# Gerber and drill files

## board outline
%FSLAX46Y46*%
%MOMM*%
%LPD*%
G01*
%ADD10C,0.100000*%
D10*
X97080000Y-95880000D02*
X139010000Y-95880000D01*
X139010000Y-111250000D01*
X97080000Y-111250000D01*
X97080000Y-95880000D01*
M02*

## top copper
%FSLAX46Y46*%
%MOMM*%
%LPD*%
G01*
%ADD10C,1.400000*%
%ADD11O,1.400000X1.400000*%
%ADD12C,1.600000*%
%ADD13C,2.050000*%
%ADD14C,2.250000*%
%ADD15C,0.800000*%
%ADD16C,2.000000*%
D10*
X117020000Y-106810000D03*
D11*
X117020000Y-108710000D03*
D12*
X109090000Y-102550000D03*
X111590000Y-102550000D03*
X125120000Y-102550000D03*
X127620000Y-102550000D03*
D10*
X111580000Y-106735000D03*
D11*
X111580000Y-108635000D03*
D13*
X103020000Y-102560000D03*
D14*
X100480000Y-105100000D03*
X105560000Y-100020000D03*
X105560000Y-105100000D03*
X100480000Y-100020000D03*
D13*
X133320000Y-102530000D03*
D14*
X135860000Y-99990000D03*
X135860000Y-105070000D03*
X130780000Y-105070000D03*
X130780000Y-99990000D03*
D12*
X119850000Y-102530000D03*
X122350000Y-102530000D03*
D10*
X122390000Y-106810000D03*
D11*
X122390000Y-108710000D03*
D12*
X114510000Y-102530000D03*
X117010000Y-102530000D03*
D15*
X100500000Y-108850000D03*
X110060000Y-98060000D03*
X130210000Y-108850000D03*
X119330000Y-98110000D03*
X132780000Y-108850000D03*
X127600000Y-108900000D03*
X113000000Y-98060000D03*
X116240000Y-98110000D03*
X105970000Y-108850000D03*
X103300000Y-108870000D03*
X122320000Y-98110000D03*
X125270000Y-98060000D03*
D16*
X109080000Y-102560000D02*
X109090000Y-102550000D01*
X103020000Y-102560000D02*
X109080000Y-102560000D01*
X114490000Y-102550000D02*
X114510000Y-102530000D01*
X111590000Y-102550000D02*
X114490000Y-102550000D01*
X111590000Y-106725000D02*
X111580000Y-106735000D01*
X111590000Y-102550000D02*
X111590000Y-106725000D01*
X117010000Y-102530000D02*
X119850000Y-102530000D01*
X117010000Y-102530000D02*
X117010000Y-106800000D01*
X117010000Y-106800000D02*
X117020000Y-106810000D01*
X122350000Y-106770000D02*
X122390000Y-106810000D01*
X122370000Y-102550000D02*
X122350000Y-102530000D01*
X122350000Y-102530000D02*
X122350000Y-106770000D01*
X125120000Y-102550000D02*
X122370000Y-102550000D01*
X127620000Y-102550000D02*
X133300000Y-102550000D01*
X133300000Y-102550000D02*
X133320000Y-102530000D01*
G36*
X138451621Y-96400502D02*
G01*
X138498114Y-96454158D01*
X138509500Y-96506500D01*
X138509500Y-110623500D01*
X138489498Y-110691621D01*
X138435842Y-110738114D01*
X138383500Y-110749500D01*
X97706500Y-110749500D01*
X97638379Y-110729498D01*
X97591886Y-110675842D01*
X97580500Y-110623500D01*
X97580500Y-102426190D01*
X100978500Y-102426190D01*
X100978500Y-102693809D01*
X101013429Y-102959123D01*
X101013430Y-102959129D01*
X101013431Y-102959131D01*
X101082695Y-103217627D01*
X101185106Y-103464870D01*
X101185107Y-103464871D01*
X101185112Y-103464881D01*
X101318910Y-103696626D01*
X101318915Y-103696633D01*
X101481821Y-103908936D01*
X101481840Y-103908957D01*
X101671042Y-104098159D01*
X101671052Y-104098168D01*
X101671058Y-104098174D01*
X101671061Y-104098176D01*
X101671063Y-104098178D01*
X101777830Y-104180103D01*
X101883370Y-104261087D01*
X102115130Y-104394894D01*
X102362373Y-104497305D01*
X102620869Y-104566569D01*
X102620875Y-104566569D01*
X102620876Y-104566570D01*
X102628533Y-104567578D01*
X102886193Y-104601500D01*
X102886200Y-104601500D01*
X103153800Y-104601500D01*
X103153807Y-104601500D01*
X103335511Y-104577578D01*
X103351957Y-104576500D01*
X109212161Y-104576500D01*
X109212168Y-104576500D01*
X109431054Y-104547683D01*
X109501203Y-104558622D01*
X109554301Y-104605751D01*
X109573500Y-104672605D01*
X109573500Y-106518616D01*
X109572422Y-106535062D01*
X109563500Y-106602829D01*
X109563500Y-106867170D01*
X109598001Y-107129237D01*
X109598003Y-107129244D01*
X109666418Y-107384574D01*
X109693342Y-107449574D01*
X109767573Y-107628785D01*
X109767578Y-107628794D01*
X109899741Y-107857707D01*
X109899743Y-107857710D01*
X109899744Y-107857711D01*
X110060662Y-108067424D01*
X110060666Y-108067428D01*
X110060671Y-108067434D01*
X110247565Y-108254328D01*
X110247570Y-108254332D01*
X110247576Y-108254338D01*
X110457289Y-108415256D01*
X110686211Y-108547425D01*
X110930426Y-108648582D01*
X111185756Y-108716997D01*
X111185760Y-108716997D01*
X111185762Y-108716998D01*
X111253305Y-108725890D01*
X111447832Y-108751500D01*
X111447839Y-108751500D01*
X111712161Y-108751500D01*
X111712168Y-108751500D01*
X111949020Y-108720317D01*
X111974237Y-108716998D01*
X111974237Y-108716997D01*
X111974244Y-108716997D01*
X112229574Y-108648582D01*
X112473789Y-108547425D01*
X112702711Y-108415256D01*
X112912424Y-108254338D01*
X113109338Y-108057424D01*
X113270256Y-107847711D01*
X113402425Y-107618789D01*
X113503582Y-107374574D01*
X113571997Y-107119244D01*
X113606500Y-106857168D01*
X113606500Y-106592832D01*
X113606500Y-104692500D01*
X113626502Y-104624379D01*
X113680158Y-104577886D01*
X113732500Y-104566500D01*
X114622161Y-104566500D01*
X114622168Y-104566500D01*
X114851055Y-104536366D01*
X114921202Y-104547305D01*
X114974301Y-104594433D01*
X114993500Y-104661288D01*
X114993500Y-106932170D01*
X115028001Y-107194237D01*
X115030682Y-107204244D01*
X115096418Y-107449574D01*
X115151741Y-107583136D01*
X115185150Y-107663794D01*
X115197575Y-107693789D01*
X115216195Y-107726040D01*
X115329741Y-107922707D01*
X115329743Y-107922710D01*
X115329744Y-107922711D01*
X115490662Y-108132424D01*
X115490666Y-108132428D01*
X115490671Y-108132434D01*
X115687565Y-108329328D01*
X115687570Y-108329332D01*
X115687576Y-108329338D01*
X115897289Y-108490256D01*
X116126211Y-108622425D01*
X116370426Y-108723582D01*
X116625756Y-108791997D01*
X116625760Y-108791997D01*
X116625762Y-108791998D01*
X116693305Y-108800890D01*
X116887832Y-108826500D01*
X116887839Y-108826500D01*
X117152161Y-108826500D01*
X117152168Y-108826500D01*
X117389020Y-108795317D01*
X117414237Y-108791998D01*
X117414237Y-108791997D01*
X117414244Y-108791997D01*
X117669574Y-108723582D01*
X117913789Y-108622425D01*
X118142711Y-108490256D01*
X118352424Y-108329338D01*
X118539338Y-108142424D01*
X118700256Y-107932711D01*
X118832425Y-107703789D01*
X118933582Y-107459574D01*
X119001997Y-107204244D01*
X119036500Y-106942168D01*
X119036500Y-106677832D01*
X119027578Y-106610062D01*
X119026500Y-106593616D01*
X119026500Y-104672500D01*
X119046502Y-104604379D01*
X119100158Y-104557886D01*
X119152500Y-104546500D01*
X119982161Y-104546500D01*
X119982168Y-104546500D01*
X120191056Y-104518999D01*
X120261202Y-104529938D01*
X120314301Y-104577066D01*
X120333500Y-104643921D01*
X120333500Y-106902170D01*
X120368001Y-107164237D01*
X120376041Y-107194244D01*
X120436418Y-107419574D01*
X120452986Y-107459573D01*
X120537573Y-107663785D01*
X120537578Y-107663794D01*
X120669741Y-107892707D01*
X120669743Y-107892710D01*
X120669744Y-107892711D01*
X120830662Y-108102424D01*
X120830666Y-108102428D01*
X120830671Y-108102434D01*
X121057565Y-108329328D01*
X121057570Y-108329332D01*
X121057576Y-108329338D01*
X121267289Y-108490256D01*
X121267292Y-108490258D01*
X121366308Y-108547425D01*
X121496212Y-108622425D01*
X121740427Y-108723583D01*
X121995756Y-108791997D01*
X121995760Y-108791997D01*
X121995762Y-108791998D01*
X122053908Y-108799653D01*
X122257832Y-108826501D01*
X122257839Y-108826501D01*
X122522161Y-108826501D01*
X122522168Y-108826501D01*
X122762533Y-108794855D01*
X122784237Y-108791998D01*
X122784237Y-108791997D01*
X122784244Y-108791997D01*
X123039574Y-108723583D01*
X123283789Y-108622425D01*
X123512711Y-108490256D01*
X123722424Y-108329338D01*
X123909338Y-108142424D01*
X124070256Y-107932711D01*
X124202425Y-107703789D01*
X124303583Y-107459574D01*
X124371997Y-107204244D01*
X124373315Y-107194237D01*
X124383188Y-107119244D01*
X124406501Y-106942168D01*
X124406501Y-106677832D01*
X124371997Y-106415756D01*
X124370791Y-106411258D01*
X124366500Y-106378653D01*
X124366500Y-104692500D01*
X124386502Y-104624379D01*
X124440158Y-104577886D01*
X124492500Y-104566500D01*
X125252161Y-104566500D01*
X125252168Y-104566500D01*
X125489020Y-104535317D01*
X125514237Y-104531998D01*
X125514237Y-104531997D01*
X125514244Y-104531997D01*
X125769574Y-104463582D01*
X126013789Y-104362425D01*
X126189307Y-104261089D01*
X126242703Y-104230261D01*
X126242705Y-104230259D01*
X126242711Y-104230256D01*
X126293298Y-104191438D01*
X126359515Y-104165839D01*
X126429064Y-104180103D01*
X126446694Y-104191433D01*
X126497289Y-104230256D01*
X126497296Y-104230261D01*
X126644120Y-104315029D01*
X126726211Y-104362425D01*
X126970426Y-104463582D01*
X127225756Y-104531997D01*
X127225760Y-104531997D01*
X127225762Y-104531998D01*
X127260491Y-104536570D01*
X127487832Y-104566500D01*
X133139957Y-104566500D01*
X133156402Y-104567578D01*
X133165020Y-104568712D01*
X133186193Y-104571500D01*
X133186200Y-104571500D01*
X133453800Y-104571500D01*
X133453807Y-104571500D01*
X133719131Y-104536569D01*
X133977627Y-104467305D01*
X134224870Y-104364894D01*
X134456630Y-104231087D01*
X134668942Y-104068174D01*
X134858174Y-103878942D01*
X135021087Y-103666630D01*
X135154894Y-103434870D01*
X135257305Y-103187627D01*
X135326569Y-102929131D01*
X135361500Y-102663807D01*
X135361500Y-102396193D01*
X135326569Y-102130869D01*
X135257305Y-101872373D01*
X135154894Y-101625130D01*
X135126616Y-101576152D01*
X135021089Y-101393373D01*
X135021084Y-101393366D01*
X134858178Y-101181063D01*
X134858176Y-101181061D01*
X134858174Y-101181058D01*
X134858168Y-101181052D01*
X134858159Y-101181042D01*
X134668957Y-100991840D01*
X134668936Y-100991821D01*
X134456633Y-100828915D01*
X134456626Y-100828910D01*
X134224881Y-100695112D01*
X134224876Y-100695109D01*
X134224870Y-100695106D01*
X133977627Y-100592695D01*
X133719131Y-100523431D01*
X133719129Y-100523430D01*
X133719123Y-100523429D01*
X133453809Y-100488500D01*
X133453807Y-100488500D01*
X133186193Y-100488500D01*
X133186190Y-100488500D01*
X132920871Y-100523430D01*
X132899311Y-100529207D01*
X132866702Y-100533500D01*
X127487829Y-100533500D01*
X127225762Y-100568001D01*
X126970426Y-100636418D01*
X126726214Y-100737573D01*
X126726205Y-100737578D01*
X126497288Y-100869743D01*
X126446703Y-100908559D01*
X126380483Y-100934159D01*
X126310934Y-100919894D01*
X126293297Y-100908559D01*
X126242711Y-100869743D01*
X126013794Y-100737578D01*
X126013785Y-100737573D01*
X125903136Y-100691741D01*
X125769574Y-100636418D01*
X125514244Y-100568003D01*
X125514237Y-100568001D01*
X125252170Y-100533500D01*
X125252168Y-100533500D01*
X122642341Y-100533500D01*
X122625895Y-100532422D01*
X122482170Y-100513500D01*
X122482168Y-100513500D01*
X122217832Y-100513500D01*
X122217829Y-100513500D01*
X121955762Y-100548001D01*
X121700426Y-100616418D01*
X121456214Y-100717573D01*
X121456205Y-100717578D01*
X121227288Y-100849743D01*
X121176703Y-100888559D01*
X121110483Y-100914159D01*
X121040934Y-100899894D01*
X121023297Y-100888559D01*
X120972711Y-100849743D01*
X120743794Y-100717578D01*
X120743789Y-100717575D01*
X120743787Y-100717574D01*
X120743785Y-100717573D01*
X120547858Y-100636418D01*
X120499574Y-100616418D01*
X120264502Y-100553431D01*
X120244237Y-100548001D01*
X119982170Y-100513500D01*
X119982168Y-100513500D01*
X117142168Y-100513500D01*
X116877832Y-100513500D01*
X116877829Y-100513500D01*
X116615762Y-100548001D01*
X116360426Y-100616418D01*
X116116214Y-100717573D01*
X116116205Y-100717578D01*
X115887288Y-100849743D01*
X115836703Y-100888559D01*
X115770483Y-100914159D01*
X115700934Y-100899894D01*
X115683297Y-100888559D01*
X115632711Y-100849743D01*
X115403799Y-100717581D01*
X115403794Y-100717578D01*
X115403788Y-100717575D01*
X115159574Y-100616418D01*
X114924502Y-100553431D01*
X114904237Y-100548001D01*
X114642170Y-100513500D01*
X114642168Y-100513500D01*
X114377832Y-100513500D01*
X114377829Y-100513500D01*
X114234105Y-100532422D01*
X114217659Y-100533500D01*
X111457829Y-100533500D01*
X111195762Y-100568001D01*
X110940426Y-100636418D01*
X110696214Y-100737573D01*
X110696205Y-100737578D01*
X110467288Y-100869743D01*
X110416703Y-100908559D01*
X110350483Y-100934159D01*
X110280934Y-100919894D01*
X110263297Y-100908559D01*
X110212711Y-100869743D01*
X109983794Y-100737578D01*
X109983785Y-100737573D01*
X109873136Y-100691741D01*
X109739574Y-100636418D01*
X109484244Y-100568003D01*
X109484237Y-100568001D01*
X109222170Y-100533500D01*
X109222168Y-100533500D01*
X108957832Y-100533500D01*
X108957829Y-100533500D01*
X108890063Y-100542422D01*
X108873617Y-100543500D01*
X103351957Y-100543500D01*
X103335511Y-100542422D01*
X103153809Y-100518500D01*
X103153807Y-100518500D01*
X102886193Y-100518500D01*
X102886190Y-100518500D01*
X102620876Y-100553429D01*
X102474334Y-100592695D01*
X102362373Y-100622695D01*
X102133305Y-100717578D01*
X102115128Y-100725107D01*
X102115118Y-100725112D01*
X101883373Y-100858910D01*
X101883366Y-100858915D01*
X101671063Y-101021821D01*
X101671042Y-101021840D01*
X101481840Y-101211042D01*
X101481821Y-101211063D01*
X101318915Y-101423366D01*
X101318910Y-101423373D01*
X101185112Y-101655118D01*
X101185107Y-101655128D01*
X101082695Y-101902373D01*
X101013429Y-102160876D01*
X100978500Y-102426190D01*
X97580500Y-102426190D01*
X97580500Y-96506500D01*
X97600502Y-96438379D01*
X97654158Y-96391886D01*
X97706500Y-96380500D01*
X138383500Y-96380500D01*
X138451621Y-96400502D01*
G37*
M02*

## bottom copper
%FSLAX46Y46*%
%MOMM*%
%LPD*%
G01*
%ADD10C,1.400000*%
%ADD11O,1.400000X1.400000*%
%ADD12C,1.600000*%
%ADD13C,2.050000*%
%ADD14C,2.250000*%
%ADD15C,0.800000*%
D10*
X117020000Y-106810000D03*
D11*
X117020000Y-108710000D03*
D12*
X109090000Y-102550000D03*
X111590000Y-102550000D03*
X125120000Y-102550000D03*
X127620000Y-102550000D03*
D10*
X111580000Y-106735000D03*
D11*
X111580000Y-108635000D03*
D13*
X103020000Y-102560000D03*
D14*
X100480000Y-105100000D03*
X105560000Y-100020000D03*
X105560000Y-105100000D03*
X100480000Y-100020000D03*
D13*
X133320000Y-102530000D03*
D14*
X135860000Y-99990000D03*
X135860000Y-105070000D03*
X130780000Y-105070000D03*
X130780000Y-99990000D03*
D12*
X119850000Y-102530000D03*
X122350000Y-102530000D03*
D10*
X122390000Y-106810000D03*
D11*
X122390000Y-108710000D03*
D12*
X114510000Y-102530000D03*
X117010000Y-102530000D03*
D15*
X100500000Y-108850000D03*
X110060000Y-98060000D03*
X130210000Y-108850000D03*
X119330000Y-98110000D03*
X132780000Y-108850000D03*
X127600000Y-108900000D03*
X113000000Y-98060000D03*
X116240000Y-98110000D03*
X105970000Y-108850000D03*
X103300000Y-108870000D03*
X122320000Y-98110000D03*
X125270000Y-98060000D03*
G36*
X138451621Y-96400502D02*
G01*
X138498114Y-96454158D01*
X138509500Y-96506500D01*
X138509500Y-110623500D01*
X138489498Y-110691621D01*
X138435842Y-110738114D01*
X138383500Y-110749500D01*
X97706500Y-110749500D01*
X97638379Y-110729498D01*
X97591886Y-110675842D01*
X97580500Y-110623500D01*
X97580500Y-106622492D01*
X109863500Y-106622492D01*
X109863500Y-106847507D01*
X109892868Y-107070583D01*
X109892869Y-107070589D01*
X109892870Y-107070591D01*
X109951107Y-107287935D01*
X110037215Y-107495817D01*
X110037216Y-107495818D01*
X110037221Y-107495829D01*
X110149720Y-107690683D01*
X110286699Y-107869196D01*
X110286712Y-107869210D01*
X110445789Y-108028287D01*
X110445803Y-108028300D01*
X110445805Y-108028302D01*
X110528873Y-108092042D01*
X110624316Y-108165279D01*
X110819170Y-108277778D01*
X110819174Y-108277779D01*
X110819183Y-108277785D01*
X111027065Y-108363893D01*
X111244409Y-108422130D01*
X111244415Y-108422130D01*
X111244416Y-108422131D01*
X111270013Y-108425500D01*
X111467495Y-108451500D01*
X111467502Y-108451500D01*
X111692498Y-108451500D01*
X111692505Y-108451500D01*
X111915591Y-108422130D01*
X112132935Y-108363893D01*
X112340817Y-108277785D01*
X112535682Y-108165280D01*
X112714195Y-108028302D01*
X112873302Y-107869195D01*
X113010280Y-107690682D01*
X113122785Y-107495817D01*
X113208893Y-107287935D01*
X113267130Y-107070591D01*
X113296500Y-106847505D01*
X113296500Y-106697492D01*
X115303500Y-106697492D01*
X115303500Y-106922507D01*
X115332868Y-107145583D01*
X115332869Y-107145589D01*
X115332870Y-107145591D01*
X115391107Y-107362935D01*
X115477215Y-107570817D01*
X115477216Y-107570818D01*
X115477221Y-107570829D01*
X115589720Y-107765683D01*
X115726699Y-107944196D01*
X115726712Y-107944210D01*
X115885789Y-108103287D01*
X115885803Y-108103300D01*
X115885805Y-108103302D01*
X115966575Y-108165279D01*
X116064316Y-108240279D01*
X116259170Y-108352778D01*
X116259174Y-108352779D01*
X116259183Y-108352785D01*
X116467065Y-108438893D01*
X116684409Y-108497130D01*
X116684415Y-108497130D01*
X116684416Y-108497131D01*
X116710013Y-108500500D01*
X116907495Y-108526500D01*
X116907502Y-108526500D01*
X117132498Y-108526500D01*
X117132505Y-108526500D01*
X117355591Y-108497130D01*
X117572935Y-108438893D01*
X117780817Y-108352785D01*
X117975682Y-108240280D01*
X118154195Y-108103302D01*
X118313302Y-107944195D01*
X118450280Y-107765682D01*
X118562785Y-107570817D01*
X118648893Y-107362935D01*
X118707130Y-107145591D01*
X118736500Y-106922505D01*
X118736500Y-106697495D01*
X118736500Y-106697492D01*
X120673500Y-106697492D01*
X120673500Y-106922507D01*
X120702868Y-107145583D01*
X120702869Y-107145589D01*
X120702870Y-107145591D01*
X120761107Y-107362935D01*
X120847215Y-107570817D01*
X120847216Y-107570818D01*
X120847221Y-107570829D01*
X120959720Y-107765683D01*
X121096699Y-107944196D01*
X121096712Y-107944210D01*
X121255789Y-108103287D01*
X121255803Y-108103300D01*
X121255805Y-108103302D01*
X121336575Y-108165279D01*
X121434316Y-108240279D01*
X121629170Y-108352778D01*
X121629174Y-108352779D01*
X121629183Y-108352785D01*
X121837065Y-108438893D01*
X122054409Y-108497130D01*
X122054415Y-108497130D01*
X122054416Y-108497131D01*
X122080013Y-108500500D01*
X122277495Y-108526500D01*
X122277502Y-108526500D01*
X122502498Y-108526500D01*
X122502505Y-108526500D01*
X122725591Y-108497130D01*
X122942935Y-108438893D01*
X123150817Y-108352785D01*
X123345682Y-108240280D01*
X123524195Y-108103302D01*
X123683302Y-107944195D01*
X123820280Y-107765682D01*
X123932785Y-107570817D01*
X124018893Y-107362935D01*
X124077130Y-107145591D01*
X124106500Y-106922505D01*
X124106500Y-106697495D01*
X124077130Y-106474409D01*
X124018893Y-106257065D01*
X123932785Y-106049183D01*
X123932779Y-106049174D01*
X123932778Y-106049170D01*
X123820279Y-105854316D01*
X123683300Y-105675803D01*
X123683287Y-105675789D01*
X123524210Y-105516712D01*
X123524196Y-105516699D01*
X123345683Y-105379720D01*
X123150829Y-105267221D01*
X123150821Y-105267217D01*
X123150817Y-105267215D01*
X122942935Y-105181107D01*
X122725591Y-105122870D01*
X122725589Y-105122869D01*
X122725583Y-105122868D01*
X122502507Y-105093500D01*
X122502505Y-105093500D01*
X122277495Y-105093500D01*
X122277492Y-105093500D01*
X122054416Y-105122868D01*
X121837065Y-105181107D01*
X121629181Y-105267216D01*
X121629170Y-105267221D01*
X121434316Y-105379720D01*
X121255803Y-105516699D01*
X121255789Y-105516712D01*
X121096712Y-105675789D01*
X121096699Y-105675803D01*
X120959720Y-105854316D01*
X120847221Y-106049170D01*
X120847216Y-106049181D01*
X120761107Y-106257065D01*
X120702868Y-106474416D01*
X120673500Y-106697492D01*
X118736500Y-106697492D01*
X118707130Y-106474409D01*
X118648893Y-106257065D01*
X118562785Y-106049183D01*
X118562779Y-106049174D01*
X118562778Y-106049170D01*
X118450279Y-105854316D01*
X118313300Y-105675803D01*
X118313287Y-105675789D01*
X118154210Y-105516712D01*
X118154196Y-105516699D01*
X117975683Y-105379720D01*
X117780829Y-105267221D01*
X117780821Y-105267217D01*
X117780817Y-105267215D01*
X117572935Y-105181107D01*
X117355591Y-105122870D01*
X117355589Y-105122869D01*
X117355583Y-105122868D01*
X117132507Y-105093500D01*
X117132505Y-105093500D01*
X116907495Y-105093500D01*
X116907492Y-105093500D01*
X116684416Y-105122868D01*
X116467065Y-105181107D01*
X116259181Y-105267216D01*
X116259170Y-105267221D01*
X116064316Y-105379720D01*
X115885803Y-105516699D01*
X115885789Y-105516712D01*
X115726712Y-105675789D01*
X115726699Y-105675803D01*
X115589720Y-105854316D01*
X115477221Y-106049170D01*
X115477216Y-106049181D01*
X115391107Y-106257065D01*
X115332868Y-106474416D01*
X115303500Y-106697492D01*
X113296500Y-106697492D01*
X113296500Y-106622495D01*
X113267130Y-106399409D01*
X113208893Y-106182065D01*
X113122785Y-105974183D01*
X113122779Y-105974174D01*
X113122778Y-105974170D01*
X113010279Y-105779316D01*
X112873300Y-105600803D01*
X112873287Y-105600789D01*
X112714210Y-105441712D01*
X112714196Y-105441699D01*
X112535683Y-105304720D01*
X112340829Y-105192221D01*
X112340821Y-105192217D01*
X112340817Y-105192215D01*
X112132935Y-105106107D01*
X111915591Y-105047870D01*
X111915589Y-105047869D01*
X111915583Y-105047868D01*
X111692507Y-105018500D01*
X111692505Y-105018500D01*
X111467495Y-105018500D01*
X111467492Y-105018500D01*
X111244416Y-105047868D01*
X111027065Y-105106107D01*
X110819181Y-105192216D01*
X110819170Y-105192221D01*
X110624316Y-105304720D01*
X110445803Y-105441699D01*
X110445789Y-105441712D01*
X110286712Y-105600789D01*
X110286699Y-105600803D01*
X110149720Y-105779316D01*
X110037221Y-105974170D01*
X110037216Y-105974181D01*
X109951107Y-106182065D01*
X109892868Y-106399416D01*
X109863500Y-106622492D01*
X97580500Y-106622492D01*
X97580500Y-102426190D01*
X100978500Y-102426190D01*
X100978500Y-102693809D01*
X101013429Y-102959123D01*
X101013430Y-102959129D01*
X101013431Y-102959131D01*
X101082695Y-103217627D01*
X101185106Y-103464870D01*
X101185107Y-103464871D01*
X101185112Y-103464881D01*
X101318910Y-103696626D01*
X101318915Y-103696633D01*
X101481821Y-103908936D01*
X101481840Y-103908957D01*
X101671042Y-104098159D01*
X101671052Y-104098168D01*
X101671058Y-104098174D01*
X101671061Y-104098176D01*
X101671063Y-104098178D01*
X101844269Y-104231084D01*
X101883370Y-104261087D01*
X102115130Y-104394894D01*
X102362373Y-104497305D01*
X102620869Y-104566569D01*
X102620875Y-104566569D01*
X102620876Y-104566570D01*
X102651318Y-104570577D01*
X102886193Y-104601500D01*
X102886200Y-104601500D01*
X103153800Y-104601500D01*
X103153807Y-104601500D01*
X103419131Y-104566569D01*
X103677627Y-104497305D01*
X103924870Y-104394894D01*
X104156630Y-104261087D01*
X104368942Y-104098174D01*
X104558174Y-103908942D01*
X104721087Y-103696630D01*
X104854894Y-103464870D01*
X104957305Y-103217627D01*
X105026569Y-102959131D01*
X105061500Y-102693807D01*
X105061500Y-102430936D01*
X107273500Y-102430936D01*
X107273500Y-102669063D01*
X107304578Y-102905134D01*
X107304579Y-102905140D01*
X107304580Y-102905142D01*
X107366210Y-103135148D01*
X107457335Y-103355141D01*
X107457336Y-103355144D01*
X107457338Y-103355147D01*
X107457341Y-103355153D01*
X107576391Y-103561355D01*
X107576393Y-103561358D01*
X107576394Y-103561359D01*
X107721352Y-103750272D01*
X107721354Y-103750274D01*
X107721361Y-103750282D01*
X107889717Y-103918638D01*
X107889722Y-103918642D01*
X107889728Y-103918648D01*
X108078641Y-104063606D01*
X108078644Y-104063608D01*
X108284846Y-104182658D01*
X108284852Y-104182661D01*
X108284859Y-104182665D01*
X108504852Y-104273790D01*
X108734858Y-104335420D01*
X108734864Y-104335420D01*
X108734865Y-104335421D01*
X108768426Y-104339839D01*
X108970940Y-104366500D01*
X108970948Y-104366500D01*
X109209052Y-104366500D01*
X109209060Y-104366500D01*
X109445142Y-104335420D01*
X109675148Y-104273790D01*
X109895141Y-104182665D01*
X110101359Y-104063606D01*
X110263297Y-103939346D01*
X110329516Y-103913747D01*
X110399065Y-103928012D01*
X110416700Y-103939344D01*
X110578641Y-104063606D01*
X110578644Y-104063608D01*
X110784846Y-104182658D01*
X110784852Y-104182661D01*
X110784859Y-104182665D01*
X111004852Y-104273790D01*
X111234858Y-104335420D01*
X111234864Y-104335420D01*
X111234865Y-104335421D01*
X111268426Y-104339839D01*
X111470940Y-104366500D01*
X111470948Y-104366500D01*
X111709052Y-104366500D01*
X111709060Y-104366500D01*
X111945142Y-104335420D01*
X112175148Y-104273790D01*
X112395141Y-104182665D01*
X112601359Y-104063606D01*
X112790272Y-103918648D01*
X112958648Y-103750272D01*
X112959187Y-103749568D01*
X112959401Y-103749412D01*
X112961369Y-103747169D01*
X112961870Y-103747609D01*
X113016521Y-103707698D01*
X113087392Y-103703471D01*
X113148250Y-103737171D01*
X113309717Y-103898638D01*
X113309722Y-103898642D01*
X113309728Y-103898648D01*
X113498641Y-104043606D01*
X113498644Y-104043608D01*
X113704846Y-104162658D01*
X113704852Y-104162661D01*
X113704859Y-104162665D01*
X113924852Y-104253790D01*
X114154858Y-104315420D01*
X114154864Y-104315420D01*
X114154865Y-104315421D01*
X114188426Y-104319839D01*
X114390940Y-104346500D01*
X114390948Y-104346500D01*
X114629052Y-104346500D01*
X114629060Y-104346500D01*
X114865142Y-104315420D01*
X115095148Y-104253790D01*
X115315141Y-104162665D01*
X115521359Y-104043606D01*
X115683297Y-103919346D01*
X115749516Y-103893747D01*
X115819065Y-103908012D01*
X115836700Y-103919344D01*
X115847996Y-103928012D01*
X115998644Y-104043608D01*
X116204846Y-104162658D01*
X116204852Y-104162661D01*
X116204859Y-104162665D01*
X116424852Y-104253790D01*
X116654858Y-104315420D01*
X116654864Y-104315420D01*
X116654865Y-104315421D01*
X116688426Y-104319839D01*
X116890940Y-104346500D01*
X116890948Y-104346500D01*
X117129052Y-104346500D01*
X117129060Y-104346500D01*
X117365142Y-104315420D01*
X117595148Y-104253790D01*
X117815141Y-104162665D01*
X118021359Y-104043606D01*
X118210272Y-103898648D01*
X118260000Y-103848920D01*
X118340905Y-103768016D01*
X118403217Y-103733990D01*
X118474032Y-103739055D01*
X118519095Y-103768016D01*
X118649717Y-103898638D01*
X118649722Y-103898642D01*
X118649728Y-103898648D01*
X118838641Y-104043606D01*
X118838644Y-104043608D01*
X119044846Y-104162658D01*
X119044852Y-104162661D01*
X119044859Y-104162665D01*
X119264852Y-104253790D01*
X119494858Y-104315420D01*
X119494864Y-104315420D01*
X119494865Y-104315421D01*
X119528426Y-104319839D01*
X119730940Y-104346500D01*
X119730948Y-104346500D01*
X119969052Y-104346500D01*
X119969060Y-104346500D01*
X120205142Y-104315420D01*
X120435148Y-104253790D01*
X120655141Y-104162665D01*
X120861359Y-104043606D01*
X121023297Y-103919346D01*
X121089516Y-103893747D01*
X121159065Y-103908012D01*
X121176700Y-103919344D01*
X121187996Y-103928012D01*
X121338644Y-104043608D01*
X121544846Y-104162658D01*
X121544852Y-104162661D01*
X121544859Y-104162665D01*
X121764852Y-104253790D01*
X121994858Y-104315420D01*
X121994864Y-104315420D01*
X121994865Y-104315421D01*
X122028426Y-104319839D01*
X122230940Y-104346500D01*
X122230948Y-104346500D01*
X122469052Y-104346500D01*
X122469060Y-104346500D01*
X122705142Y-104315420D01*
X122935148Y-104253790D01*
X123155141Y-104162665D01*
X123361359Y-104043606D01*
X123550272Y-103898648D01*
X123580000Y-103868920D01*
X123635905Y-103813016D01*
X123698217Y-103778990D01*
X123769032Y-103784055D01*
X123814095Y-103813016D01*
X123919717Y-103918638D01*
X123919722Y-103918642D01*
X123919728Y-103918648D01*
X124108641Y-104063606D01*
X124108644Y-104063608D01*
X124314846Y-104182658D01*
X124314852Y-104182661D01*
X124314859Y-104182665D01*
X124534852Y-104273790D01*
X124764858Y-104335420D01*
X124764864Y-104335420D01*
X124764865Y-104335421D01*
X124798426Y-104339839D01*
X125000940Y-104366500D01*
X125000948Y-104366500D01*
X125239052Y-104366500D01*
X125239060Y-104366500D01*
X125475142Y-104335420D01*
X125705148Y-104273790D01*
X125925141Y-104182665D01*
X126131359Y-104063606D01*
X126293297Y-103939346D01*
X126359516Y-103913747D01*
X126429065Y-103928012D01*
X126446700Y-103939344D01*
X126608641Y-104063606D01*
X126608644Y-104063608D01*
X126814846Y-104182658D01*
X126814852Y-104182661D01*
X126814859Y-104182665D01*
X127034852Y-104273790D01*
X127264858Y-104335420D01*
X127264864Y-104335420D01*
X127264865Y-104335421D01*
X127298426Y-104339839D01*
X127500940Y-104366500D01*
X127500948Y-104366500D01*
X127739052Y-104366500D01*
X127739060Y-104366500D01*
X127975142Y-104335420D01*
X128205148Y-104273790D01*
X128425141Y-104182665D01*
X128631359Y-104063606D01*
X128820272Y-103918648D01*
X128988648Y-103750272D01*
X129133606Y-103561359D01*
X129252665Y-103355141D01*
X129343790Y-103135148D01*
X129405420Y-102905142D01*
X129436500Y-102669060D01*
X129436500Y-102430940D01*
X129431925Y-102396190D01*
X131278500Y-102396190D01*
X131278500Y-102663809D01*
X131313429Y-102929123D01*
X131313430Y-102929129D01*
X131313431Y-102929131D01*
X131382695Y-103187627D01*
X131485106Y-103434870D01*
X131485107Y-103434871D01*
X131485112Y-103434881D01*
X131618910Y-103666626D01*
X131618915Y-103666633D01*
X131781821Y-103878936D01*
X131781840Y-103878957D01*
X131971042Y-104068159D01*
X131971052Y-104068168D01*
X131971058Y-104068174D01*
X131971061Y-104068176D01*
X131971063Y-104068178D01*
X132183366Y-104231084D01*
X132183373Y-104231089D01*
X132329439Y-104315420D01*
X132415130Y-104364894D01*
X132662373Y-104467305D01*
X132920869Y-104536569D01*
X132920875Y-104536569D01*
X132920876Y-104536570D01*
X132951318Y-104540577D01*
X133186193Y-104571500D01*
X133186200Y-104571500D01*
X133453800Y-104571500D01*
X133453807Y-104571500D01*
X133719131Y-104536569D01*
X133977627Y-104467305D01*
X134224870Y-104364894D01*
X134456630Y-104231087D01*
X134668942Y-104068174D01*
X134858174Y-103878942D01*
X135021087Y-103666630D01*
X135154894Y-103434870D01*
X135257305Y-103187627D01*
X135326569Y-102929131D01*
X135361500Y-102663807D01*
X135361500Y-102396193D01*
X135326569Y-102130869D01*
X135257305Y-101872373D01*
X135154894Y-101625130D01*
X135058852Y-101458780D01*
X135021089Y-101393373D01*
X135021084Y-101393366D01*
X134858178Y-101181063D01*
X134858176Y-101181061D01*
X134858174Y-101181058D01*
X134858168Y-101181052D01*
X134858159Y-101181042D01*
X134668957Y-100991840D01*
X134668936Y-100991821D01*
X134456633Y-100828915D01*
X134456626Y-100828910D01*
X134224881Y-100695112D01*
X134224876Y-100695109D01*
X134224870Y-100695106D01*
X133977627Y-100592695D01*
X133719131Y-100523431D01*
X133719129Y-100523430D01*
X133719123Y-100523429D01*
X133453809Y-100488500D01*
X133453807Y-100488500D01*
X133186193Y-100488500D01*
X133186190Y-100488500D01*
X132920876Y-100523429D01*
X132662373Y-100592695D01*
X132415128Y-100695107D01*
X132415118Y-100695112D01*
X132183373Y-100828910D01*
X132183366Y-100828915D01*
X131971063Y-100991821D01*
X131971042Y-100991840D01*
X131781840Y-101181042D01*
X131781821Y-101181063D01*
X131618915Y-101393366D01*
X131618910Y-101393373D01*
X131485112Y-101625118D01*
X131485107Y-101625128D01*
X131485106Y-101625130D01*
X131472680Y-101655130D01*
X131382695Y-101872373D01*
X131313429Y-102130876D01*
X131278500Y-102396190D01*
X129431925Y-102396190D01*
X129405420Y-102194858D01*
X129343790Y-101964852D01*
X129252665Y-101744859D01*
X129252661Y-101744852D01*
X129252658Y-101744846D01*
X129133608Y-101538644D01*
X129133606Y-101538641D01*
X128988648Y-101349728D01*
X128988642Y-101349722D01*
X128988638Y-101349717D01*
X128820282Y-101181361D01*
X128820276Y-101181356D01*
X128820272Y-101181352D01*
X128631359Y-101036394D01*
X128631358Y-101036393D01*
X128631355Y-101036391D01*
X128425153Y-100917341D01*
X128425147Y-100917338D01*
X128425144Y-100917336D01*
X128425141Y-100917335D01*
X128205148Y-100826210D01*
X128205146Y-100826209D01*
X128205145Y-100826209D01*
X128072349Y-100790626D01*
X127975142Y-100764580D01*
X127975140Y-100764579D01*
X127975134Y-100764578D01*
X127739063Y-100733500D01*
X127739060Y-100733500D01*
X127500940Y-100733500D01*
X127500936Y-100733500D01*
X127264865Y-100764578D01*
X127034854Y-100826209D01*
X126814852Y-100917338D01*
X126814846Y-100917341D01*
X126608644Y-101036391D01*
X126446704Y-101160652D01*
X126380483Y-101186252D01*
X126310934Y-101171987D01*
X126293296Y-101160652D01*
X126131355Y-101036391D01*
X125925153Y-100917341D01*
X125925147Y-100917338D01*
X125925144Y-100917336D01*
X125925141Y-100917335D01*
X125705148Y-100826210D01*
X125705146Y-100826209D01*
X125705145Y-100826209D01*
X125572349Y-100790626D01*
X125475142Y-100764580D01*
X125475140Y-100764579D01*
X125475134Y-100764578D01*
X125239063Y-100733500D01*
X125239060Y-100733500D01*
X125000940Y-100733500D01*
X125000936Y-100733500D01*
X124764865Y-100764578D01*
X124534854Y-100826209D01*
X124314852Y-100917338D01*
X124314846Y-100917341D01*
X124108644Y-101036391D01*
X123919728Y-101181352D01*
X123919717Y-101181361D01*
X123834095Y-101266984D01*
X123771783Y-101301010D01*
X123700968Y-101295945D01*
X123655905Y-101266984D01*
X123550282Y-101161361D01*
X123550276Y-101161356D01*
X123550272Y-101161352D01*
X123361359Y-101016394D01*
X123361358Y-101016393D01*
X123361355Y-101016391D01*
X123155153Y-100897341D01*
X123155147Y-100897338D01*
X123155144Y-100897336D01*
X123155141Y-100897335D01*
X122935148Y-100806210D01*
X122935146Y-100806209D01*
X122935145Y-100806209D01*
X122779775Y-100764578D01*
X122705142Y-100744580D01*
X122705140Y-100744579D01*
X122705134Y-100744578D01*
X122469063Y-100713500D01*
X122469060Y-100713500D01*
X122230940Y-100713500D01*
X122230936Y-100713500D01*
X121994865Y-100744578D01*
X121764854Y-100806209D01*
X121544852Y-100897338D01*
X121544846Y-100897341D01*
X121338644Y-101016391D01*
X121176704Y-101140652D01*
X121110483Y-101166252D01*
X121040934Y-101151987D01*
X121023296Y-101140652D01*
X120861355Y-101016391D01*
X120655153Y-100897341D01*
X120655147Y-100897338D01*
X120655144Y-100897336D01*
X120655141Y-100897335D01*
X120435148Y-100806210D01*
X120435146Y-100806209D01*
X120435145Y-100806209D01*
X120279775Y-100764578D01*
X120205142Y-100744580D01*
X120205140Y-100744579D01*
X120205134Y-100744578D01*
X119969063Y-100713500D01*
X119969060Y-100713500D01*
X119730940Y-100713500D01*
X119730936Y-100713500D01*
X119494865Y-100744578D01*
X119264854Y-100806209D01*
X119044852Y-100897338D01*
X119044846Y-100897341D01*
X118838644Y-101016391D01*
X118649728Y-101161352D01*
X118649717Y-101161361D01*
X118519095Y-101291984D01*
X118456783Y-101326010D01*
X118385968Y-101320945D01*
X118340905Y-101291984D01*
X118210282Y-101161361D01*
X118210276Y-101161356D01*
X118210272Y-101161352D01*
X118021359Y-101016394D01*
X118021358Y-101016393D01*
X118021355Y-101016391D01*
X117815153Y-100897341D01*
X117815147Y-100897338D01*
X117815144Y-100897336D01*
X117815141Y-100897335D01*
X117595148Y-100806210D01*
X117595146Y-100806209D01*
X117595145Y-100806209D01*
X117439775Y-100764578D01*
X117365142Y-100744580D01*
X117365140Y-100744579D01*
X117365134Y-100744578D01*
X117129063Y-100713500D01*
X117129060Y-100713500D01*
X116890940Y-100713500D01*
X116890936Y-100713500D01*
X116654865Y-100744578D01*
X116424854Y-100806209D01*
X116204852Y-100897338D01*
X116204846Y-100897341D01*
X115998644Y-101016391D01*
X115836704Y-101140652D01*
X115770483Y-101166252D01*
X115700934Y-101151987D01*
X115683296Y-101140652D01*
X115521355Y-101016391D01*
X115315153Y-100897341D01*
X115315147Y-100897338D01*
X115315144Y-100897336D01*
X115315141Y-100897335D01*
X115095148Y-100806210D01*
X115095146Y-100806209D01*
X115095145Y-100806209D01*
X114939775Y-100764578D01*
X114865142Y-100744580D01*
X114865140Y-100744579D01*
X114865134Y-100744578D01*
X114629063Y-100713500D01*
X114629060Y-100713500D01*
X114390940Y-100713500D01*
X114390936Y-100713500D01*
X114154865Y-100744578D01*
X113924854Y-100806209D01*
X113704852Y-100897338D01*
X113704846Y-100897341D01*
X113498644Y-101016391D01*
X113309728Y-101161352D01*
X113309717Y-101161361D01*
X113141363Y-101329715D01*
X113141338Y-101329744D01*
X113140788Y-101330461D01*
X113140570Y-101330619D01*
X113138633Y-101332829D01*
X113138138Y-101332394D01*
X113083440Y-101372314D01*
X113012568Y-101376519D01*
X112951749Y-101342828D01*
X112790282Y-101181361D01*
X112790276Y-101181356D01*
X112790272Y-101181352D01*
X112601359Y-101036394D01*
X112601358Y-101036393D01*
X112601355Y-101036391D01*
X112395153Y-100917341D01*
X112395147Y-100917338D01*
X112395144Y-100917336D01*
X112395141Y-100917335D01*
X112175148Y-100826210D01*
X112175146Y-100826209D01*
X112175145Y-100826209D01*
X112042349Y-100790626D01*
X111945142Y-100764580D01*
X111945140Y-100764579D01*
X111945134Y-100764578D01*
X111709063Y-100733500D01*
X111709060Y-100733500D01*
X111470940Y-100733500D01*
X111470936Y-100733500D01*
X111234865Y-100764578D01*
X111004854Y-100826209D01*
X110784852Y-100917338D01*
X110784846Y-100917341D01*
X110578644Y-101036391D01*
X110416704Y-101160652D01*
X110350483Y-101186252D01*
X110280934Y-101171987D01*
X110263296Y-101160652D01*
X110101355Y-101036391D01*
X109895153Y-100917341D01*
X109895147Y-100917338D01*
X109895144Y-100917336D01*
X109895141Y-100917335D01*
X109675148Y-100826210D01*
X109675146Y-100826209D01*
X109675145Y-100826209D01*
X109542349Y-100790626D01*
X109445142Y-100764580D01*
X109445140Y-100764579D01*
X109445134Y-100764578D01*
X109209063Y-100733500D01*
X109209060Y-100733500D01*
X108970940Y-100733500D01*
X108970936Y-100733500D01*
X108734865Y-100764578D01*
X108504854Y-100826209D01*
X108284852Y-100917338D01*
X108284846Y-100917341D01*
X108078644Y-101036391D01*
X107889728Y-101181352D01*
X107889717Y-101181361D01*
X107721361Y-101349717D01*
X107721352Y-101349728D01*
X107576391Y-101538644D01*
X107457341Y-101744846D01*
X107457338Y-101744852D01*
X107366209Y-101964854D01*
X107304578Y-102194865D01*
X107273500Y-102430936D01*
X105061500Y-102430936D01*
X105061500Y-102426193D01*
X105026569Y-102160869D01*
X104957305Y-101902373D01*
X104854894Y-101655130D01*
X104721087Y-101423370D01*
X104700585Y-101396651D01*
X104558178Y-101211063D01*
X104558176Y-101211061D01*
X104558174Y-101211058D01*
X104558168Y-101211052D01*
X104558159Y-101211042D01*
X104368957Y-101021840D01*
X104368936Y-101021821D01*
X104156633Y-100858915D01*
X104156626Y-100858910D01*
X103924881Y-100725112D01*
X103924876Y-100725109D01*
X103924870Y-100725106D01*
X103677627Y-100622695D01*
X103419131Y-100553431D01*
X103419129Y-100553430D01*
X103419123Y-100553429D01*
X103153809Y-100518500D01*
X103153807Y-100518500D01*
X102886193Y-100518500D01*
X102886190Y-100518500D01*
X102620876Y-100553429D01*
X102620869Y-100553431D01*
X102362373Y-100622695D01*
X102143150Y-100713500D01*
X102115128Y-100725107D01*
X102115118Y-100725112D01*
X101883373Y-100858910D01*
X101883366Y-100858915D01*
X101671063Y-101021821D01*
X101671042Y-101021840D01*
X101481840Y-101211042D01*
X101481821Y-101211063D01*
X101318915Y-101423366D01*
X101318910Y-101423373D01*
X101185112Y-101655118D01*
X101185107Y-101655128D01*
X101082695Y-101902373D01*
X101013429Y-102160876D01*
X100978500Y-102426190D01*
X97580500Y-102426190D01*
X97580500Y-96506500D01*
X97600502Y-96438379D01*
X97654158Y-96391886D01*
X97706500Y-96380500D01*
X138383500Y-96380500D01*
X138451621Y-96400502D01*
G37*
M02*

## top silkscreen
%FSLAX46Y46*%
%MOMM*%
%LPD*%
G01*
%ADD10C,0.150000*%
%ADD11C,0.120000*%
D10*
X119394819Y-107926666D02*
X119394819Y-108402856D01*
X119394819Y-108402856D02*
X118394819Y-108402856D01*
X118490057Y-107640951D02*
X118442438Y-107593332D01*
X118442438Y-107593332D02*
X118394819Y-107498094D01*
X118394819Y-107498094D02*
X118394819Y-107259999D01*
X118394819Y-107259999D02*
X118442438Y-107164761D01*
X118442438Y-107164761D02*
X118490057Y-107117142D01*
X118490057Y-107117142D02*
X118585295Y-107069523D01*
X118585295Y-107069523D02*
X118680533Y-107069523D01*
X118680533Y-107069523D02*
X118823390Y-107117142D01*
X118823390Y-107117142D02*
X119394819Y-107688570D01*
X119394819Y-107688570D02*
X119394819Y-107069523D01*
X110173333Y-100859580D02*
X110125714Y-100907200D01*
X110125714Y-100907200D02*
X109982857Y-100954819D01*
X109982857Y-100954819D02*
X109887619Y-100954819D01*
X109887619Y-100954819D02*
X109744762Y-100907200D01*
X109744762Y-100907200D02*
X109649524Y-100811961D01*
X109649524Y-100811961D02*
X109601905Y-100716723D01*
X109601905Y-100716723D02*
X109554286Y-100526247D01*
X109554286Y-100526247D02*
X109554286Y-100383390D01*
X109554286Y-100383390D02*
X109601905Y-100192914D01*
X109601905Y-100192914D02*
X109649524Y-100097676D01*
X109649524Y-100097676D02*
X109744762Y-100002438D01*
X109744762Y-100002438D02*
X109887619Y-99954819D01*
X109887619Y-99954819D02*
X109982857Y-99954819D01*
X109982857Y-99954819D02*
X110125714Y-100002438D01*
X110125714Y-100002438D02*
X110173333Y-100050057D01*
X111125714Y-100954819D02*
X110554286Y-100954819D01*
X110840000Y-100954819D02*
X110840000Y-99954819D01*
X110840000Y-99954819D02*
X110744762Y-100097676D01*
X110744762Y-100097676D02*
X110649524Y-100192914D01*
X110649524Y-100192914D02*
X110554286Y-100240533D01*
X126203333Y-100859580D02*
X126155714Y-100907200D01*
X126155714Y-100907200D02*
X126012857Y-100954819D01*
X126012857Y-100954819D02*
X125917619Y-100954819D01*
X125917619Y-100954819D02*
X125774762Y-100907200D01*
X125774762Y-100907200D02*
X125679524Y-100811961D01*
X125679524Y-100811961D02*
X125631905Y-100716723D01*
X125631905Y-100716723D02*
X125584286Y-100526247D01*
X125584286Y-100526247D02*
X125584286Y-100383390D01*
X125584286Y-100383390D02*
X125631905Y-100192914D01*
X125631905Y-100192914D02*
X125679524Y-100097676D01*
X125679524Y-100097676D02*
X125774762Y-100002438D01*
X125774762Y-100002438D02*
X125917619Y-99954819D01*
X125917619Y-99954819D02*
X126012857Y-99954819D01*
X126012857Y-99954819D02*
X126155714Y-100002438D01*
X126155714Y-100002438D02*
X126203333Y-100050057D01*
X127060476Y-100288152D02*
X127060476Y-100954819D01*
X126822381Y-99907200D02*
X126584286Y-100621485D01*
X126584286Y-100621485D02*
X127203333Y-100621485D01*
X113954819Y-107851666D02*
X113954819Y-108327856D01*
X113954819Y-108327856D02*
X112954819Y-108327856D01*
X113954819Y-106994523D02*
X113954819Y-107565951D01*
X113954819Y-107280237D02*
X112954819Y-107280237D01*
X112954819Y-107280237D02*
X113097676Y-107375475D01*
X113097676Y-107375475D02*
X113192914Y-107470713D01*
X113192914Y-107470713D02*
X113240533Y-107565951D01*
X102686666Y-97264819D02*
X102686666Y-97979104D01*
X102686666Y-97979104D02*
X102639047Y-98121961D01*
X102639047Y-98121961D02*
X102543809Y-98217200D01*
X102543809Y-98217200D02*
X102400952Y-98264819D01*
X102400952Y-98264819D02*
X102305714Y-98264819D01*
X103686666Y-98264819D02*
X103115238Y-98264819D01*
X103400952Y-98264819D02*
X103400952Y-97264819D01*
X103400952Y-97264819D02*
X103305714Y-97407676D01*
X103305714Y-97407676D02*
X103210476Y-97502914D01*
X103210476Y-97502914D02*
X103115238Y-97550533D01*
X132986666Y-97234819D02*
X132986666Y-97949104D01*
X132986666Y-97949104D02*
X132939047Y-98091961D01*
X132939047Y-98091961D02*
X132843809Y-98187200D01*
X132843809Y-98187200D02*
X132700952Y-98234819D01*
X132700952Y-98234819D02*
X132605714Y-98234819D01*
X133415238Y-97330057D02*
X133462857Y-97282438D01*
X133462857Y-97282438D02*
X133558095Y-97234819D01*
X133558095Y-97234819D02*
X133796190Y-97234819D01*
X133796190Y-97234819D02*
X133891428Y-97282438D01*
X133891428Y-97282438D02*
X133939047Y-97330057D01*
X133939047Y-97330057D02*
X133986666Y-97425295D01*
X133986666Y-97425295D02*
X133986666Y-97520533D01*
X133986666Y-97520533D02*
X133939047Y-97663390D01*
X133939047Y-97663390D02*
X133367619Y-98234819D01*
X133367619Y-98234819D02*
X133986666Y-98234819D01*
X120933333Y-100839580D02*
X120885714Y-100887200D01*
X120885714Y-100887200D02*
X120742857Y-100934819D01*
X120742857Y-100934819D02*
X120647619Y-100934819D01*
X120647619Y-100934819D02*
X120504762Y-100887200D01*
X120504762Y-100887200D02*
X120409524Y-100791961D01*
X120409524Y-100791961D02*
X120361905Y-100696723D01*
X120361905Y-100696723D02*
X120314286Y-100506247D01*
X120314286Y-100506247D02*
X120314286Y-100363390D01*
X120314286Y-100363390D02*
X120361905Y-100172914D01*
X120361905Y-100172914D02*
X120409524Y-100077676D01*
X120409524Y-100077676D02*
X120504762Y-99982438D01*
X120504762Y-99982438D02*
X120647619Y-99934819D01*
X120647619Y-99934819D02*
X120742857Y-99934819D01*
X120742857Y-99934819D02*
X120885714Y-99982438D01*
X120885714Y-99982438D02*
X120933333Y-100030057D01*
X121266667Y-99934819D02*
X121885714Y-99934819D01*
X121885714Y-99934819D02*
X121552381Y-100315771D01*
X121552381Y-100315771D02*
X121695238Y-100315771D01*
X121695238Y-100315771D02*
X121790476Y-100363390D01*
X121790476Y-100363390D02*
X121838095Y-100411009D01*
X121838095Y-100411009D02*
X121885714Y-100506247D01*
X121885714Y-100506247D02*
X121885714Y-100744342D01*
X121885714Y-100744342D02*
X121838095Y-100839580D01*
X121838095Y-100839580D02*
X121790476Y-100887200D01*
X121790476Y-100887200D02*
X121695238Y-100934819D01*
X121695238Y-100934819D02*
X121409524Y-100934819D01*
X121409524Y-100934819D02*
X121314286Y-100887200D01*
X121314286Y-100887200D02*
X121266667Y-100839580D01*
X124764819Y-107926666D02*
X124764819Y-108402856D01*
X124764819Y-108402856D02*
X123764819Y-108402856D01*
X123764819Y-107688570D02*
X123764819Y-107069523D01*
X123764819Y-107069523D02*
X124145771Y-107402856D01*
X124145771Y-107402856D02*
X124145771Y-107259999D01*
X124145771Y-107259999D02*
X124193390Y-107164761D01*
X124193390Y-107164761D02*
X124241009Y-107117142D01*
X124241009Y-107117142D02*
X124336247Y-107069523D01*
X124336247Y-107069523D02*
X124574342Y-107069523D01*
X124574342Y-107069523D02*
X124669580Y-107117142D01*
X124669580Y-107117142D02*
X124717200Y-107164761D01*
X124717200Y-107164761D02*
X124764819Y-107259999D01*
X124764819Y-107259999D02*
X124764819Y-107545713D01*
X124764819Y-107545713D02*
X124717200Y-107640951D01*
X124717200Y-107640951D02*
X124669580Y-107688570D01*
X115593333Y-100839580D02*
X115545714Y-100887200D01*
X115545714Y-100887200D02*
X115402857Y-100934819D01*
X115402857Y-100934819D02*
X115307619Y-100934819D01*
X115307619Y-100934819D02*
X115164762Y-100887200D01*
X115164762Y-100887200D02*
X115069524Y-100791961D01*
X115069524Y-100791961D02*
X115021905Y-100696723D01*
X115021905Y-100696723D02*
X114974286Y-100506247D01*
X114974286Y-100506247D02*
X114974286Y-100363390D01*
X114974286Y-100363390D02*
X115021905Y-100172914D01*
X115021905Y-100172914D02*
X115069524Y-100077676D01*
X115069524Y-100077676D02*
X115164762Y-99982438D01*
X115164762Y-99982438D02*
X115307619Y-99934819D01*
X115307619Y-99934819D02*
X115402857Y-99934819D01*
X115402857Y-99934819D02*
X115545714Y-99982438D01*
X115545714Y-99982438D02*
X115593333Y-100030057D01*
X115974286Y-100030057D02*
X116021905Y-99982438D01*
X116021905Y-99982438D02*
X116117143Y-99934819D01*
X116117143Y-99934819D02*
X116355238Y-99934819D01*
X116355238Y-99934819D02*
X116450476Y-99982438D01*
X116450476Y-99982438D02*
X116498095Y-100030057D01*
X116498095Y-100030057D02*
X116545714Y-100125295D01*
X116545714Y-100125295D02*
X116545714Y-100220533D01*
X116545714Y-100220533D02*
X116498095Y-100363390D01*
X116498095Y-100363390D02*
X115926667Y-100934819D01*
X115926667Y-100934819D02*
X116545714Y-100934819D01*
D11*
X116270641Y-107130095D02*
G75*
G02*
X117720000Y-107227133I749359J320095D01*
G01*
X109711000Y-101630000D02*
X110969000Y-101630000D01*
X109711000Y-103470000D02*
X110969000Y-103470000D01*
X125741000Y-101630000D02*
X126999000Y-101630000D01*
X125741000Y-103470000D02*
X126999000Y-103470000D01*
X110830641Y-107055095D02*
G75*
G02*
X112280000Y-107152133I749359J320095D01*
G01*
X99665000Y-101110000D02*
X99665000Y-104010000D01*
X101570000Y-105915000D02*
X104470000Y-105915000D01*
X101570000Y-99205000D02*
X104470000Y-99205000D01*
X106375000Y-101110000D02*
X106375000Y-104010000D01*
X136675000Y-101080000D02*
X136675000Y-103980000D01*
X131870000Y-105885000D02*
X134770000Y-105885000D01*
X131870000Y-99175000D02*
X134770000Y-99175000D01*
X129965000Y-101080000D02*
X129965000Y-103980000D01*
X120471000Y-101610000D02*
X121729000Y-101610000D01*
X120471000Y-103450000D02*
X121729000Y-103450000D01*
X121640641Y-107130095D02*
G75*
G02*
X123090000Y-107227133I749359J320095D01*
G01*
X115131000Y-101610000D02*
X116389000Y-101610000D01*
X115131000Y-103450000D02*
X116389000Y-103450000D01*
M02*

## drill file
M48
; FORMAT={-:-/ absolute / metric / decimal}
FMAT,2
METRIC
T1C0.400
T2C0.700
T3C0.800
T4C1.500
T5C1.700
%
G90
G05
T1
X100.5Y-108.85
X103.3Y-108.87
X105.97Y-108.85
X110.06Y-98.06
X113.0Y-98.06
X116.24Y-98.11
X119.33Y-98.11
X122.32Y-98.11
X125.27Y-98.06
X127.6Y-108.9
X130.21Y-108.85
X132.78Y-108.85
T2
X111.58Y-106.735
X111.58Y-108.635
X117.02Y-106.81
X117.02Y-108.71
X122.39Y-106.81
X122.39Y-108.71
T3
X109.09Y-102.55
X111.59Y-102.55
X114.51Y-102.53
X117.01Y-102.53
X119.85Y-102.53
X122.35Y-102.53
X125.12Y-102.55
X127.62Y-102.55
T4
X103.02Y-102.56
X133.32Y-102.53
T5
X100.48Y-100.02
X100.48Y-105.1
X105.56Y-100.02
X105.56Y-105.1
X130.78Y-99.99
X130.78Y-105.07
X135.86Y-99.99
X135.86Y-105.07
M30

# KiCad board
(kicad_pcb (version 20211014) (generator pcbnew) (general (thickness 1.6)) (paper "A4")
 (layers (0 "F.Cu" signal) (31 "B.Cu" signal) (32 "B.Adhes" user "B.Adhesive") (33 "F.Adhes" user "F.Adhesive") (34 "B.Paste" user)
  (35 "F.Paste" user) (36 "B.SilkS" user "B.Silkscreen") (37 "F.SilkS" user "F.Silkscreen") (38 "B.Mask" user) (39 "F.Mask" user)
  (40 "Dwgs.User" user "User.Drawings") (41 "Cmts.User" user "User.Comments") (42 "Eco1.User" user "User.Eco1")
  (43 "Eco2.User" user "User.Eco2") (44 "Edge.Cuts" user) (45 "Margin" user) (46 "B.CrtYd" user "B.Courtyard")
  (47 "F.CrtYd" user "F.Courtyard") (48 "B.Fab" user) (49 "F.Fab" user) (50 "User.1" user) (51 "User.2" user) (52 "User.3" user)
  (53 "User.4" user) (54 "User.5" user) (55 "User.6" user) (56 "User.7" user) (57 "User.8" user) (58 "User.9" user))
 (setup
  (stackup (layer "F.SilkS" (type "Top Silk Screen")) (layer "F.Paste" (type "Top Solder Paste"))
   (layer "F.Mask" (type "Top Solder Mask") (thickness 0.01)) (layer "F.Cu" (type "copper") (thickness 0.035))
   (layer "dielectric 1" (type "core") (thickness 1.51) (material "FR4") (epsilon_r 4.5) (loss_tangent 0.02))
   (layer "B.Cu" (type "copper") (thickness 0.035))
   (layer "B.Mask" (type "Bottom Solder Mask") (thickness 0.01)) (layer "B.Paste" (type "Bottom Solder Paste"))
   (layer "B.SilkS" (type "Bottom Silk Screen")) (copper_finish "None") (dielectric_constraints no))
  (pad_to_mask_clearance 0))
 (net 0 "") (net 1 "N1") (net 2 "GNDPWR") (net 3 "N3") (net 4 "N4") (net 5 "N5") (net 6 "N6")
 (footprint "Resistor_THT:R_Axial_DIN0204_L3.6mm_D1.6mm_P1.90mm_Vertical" (layer "F.Cu") (at 117.02 106.81 -90)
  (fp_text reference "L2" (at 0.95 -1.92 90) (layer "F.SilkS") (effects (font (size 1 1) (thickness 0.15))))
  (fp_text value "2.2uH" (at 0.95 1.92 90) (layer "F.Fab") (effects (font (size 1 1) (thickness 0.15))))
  (fp_arc (start 0.320095 0.749359) (mid -0.813042 -0.054435) (end 0.417133 -0.7) (layer "F.SilkS") (width 0.12))
  (pad "1" thru_hole circle (at 0 0 270) (size 1.4 1.4) (drill 0.7) (layers *.Cu *.Mask) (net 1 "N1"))
  (pad "2" thru_hole oval (at 1.9 0 270) (size 1.4 1.4) (drill 0.7) (layers *.Cu *.Mask) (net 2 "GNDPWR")))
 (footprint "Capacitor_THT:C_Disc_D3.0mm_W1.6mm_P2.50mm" (layer "F.Cu") (at 109.09 102.55)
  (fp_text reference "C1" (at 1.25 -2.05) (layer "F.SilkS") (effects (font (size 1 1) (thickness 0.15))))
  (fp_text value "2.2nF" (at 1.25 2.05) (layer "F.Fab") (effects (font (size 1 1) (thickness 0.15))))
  (fp_line (start 0.621 -0.92) (end 1.879 -0.92) (layer "F.SilkS") (width 0.12))
  (fp_line (start 0.621 0.92) (end 1.879 0.92) (layer "F.SilkS") (width 0.12))
  (pad "1" thru_hole circle (at 0 0) (size 1.6 1.6) (drill 0.8) (layers *.Cu *.Mask) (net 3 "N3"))
  (pad "2" thru_hole circle (at 2.5 0) (size 1.6 1.6) (drill 0.8) (layers *.Cu *.Mask) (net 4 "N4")))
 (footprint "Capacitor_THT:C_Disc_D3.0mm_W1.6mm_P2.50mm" (layer "F.Cu") (at 125.12 102.55)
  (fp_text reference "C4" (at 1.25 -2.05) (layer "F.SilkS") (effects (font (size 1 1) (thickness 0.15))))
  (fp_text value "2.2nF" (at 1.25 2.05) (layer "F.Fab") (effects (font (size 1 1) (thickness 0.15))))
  (fp_line (start 0.621 -0.92) (end 1.879 -0.92) (layer "F.SilkS") (width 0.12))
  (fp_line (start 0.621 0.92) (end 1.879 0.92) (layer "F.SilkS") (width 0.12))
  (pad "1" thru_hole circle (at 0 0) (size 1.6 1.6) (drill 0.8) (layers *.Cu *.Mask) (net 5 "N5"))
  (pad "2" thru_hole circle (at 2.5 0) (size 1.6 1.6) (drill 0.8) (layers *.Cu *.Mask) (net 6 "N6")))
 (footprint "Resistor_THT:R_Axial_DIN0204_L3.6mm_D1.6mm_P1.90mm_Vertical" (layer "F.Cu") (at 111.58 106.735 -90)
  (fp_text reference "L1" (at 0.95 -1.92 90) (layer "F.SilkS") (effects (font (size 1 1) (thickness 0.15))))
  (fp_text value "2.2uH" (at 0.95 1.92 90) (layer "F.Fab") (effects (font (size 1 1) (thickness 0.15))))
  (fp_arc (start 0.320095 0.749359) (mid -0.813042 -0.054435) (end 0.417133 -0.7) (layer "F.SilkS") (width 0.12))
  (pad "1" thru_hole circle (at 0 0 270) (size 1.4 1.4) (drill 0.7) (layers *.Cu *.Mask) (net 4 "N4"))
  (pad "2" thru_hole oval (at 1.9 0 270) (size 1.4 1.4) (drill 0.7) (layers *.Cu *.Mask) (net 2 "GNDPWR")))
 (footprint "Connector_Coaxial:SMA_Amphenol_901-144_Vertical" (layer "F.Cu") (at 103.02 102.56)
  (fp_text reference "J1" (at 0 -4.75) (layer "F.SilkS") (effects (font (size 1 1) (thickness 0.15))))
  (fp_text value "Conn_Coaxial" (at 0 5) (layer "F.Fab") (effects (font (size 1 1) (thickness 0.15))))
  (fp_line (start -3.355 -1.45) (end -3.355 1.45) (layer "F.SilkS") (width 0.12))
  (fp_line (start -1.45 3.355) (end 1.45 3.355) (layer "F.SilkS") (width 0.12))
  (fp_line (start -1.45 -3.355) (end 1.45 -3.355) (layer "F.SilkS") (width 0.12))
  (fp_line (start 3.355 -1.45) (end 3.355 1.45) (layer "F.SilkS") (width 0.12))
  (pad "1" thru_hole circle (at 0 0) (size 2.05 2.05) (drill 1.5) (layers *.Cu *.Mask) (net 3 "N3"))
  (pad "2" thru_hole circle (at -2.54 2.54) (size 2.25 2.25) (drill 1.7) (layers *.Cu *.Mask) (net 2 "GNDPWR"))
  (pad "2" thru_hole circle (at 2.54 -2.54) (size 2.25 2.25) (drill 1.7) (layers *.Cu *.Mask) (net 2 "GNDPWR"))
  (pad "2" thru_hole circle (at 2.54 2.54) (size 2.25 2.25) (drill 1.7) (layers *.Cu *.Mask) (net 2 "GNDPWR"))
  (pad "2" thru_hole circle (at -2.54 -2.54) (size 2.25 2.25) (drill 1.7) (layers *.Cu *.Mask) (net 2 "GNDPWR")))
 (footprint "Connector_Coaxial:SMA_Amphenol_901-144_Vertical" (layer "F.Cu") (at 133.32 102.53)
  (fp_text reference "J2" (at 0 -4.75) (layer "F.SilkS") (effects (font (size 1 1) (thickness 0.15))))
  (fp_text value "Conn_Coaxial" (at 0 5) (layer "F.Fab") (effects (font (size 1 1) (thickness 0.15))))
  (fp_line (start 3.355 -1.45) (end 3.355 1.45) (layer "F.SilkS") (width 0.12))
  (fp_line (start -1.45 3.355) (end 1.45 3.355) (layer "F.SilkS") (width 0.12))
  (fp_line (start -1.45 -3.355) (end 1.45 -3.355) (layer "F.SilkS") (width 0.12))
  (fp_line (start -3.355 -1.45) (end -3.355 1.45) (layer "F.SilkS") (width 0.12))
  (pad "1" thru_hole circle (at 0 0) (size 2.05 2.05) (drill 1.5) (layers *.Cu *.Mask) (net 6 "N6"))
  (pad "2" thru_hole circle (at 2.54 -2.54) (size 2.25 2.25) (drill 1.7) (layers *.Cu *.Mask) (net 2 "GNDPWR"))
  (pad "2" thru_hole circle (at 2.54 2.54) (size 2.25 2.25) (drill 1.7) (layers *.Cu *.Mask) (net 2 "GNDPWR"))
  (pad "2" thru_hole circle (at -2.54 2.54) (size 2.25 2.25) (drill 1.7) (layers *.Cu *.Mask) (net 2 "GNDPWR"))
  (pad "2" thru_hole circle (at -2.54 -2.54) (size 2.25 2.25) (drill 1.7) (layers *.Cu *.Mask) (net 2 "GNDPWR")))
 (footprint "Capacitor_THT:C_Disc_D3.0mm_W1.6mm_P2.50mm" (layer "F.Cu") (at 119.85 102.53)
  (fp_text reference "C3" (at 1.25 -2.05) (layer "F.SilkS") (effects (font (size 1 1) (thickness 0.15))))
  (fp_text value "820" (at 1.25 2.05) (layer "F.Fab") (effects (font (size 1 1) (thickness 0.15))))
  (fp_line (start 0.621 -0.92) (end 1.879 -0.92) (layer "F.SilkS") (width 0.12))
  (fp_line (start 0.621 0.92) (end 1.879 0.92) (layer "F.SilkS") (width 0.12))
  (pad "1" thru_hole circle (at 0 0) (size 1.6 1.6) (drill 0.8) (layers *.Cu *.Mask) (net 1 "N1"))
  (pad "2" thru_hole circle (at 2.5 0) (size 1.6 1.6) (drill 0.8) (layers *.Cu *.Mask) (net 5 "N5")))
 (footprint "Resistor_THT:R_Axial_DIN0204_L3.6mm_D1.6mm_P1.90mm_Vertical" (layer "F.Cu") (at 122.39 106.81 -90)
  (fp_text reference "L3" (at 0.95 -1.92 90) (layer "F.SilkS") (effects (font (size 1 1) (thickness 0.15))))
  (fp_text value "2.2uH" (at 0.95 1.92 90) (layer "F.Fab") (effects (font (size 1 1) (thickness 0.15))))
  (fp_arc (start 0.320095 0.749359) (mid -0.813042 -0.054435) (end 0.417133 -0.7) (layer "F.SilkS") (width 0.12))
  (pad "1" thru_hole circle (at 0 0 270) (size 1.4 1.4) (drill 0.7) (layers *.Cu *.Mask) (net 5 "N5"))
  (pad "2" thru_hole oval (at 1.9 0 270) (size 1.4 1.4) (drill 0.7) (layers *.Cu *.Mask) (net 2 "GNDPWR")))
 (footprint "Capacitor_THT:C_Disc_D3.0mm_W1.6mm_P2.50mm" (layer "F.Cu") (at 114.51 102.53)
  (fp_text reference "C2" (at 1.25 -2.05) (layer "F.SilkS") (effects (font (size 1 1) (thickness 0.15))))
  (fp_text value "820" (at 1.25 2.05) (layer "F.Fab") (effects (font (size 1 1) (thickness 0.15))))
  (fp_line (start 0.621 -0.92) (end 1.879 -0.92) (layer "F.SilkS") (width 0.12))
  (fp_line (start 0.621 0.92) (end 1.879 0.92) (layer "F.SilkS") (width 0.12))
  (pad "1" thru_hole circle (at 0 0) (size 1.6 1.6) (drill 0.8) (layers *.Cu *.Mask) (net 4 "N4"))
  (pad "2" thru_hole circle (at 2.5 0) (size 1.6 1.6) (drill 0.8) (layers *.Cu *.Mask) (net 1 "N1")))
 (gr_rect (start 97.08 95.88) (end 139.01 111.25) (layer "Edge.Cuts") (width 0.1) (fill none))
 (segment (start 109.08 102.56) (end 109.09 102.55) (width 2) (layer "F.Cu") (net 3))
 (segment (start 103.02 102.56) (end 109.08 102.56) (width 2) (layer "F.Cu") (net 3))
 (segment (start 114.49 102.55) (end 114.51 102.53) (width 2) (layer "F.Cu") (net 4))
 (segment (start 111.59 102.55) (end 114.49 102.55) (width 2) (layer "F.Cu") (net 4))
 (segment (start 111.59 106.725) (end 111.58 106.735) (width 2) (layer "F.Cu") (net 4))
 (segment (start 111.59 102.55) (end 111.59 106.725) (width 2) (layer "F.Cu") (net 4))
 (segment (start 117.01 102.53) (end 119.85 102.53) (width 2) (layer "F.Cu") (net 1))
 (segment (start 117.01 102.53) (end 117.01 106.8) (width 2) (layer "F.Cu") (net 1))
 (segment (start 117.01 106.8) (end 117.02 106.81) (width 2) (layer "F.Cu") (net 1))
 (segment (start 122.35 106.77) (end 122.39 106.81) (width 2) (layer "F.Cu") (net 5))
 (segment (start 122.37 102.55) (end 122.35 102.53) (width 2) (layer "F.Cu") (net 5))
 (segment (start 122.35 102.53) (end 122.35 106.77) (width 2) (layer "F.Cu") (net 5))
 (segment (start 125.12 102.55) (end 122.37 102.55) (width 2) (layer "F.Cu") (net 5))
 (segment (start 127.62 102.55) (end 133.3 102.55) (width 2) (layer "F.Cu") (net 6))
 (segment (start 133.3 102.55) (end 133.32 102.53) (width 2) (layer "F.Cu") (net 6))
 (via (at 100.5 108.85) (size 0.8) (drill 0.4) (layers "F.Cu" "B.Cu") (free) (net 2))
 (via (at 110.06 98.06) (size 0.8) (drill 0.4) (layers "F.Cu" "B.Cu") (free) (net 2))
 (via (at 130.21 108.85) (size 0.8) (drill 0.4) (layers "F.Cu" "B.Cu") (free) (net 2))
 (via (at 119.33 98.11) (size 0.8) (drill 0.4) (layers "F.Cu" "B.Cu") (free) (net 2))
 (via (at 132.78 108.85) (size 0.8) (drill 0.4) (layers "F.Cu" "B.Cu") (free) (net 2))
 (via (at 127.6 108.9) (size 0.8) (drill 0.4) (layers "F.Cu" "B.Cu") (free) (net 2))
 (via (at 113 98.06) (size 0.8) (drill 0.4) (layers "F.Cu" "B.Cu") (free) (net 2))
 (via (at 116.24 98.11) (size 0.8) (drill 0.4) (layers "F.Cu" "B.Cu") (free) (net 2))
 (via (at 105.97 108.85) (size 0.8) (drill 0.4) (layers "F.Cu" "B.Cu") (free) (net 2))
 (via (at 103.3 108.87) (size 0.8) (drill 0.4) (layers "F.Cu" "B.Cu") (free) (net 2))
 (via (at 122.32 98.11) (size 0.8) (drill 0.4) (layers "F.Cu" "B.Cu") (free) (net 2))
 (via (at 125.27 98.06) (size 0.8) (drill 0.4) (layers "F.Cu" "B.Cu") (free) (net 2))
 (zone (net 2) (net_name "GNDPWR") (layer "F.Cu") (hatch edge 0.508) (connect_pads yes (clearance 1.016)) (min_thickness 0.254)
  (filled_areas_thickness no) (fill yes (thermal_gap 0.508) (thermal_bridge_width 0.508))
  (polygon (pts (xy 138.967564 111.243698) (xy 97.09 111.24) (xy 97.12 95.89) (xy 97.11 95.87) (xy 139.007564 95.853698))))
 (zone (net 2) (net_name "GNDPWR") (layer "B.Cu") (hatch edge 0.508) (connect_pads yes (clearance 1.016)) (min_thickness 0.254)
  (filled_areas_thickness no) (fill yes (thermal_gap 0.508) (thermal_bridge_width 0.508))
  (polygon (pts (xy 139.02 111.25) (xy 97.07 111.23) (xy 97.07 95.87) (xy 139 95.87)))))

